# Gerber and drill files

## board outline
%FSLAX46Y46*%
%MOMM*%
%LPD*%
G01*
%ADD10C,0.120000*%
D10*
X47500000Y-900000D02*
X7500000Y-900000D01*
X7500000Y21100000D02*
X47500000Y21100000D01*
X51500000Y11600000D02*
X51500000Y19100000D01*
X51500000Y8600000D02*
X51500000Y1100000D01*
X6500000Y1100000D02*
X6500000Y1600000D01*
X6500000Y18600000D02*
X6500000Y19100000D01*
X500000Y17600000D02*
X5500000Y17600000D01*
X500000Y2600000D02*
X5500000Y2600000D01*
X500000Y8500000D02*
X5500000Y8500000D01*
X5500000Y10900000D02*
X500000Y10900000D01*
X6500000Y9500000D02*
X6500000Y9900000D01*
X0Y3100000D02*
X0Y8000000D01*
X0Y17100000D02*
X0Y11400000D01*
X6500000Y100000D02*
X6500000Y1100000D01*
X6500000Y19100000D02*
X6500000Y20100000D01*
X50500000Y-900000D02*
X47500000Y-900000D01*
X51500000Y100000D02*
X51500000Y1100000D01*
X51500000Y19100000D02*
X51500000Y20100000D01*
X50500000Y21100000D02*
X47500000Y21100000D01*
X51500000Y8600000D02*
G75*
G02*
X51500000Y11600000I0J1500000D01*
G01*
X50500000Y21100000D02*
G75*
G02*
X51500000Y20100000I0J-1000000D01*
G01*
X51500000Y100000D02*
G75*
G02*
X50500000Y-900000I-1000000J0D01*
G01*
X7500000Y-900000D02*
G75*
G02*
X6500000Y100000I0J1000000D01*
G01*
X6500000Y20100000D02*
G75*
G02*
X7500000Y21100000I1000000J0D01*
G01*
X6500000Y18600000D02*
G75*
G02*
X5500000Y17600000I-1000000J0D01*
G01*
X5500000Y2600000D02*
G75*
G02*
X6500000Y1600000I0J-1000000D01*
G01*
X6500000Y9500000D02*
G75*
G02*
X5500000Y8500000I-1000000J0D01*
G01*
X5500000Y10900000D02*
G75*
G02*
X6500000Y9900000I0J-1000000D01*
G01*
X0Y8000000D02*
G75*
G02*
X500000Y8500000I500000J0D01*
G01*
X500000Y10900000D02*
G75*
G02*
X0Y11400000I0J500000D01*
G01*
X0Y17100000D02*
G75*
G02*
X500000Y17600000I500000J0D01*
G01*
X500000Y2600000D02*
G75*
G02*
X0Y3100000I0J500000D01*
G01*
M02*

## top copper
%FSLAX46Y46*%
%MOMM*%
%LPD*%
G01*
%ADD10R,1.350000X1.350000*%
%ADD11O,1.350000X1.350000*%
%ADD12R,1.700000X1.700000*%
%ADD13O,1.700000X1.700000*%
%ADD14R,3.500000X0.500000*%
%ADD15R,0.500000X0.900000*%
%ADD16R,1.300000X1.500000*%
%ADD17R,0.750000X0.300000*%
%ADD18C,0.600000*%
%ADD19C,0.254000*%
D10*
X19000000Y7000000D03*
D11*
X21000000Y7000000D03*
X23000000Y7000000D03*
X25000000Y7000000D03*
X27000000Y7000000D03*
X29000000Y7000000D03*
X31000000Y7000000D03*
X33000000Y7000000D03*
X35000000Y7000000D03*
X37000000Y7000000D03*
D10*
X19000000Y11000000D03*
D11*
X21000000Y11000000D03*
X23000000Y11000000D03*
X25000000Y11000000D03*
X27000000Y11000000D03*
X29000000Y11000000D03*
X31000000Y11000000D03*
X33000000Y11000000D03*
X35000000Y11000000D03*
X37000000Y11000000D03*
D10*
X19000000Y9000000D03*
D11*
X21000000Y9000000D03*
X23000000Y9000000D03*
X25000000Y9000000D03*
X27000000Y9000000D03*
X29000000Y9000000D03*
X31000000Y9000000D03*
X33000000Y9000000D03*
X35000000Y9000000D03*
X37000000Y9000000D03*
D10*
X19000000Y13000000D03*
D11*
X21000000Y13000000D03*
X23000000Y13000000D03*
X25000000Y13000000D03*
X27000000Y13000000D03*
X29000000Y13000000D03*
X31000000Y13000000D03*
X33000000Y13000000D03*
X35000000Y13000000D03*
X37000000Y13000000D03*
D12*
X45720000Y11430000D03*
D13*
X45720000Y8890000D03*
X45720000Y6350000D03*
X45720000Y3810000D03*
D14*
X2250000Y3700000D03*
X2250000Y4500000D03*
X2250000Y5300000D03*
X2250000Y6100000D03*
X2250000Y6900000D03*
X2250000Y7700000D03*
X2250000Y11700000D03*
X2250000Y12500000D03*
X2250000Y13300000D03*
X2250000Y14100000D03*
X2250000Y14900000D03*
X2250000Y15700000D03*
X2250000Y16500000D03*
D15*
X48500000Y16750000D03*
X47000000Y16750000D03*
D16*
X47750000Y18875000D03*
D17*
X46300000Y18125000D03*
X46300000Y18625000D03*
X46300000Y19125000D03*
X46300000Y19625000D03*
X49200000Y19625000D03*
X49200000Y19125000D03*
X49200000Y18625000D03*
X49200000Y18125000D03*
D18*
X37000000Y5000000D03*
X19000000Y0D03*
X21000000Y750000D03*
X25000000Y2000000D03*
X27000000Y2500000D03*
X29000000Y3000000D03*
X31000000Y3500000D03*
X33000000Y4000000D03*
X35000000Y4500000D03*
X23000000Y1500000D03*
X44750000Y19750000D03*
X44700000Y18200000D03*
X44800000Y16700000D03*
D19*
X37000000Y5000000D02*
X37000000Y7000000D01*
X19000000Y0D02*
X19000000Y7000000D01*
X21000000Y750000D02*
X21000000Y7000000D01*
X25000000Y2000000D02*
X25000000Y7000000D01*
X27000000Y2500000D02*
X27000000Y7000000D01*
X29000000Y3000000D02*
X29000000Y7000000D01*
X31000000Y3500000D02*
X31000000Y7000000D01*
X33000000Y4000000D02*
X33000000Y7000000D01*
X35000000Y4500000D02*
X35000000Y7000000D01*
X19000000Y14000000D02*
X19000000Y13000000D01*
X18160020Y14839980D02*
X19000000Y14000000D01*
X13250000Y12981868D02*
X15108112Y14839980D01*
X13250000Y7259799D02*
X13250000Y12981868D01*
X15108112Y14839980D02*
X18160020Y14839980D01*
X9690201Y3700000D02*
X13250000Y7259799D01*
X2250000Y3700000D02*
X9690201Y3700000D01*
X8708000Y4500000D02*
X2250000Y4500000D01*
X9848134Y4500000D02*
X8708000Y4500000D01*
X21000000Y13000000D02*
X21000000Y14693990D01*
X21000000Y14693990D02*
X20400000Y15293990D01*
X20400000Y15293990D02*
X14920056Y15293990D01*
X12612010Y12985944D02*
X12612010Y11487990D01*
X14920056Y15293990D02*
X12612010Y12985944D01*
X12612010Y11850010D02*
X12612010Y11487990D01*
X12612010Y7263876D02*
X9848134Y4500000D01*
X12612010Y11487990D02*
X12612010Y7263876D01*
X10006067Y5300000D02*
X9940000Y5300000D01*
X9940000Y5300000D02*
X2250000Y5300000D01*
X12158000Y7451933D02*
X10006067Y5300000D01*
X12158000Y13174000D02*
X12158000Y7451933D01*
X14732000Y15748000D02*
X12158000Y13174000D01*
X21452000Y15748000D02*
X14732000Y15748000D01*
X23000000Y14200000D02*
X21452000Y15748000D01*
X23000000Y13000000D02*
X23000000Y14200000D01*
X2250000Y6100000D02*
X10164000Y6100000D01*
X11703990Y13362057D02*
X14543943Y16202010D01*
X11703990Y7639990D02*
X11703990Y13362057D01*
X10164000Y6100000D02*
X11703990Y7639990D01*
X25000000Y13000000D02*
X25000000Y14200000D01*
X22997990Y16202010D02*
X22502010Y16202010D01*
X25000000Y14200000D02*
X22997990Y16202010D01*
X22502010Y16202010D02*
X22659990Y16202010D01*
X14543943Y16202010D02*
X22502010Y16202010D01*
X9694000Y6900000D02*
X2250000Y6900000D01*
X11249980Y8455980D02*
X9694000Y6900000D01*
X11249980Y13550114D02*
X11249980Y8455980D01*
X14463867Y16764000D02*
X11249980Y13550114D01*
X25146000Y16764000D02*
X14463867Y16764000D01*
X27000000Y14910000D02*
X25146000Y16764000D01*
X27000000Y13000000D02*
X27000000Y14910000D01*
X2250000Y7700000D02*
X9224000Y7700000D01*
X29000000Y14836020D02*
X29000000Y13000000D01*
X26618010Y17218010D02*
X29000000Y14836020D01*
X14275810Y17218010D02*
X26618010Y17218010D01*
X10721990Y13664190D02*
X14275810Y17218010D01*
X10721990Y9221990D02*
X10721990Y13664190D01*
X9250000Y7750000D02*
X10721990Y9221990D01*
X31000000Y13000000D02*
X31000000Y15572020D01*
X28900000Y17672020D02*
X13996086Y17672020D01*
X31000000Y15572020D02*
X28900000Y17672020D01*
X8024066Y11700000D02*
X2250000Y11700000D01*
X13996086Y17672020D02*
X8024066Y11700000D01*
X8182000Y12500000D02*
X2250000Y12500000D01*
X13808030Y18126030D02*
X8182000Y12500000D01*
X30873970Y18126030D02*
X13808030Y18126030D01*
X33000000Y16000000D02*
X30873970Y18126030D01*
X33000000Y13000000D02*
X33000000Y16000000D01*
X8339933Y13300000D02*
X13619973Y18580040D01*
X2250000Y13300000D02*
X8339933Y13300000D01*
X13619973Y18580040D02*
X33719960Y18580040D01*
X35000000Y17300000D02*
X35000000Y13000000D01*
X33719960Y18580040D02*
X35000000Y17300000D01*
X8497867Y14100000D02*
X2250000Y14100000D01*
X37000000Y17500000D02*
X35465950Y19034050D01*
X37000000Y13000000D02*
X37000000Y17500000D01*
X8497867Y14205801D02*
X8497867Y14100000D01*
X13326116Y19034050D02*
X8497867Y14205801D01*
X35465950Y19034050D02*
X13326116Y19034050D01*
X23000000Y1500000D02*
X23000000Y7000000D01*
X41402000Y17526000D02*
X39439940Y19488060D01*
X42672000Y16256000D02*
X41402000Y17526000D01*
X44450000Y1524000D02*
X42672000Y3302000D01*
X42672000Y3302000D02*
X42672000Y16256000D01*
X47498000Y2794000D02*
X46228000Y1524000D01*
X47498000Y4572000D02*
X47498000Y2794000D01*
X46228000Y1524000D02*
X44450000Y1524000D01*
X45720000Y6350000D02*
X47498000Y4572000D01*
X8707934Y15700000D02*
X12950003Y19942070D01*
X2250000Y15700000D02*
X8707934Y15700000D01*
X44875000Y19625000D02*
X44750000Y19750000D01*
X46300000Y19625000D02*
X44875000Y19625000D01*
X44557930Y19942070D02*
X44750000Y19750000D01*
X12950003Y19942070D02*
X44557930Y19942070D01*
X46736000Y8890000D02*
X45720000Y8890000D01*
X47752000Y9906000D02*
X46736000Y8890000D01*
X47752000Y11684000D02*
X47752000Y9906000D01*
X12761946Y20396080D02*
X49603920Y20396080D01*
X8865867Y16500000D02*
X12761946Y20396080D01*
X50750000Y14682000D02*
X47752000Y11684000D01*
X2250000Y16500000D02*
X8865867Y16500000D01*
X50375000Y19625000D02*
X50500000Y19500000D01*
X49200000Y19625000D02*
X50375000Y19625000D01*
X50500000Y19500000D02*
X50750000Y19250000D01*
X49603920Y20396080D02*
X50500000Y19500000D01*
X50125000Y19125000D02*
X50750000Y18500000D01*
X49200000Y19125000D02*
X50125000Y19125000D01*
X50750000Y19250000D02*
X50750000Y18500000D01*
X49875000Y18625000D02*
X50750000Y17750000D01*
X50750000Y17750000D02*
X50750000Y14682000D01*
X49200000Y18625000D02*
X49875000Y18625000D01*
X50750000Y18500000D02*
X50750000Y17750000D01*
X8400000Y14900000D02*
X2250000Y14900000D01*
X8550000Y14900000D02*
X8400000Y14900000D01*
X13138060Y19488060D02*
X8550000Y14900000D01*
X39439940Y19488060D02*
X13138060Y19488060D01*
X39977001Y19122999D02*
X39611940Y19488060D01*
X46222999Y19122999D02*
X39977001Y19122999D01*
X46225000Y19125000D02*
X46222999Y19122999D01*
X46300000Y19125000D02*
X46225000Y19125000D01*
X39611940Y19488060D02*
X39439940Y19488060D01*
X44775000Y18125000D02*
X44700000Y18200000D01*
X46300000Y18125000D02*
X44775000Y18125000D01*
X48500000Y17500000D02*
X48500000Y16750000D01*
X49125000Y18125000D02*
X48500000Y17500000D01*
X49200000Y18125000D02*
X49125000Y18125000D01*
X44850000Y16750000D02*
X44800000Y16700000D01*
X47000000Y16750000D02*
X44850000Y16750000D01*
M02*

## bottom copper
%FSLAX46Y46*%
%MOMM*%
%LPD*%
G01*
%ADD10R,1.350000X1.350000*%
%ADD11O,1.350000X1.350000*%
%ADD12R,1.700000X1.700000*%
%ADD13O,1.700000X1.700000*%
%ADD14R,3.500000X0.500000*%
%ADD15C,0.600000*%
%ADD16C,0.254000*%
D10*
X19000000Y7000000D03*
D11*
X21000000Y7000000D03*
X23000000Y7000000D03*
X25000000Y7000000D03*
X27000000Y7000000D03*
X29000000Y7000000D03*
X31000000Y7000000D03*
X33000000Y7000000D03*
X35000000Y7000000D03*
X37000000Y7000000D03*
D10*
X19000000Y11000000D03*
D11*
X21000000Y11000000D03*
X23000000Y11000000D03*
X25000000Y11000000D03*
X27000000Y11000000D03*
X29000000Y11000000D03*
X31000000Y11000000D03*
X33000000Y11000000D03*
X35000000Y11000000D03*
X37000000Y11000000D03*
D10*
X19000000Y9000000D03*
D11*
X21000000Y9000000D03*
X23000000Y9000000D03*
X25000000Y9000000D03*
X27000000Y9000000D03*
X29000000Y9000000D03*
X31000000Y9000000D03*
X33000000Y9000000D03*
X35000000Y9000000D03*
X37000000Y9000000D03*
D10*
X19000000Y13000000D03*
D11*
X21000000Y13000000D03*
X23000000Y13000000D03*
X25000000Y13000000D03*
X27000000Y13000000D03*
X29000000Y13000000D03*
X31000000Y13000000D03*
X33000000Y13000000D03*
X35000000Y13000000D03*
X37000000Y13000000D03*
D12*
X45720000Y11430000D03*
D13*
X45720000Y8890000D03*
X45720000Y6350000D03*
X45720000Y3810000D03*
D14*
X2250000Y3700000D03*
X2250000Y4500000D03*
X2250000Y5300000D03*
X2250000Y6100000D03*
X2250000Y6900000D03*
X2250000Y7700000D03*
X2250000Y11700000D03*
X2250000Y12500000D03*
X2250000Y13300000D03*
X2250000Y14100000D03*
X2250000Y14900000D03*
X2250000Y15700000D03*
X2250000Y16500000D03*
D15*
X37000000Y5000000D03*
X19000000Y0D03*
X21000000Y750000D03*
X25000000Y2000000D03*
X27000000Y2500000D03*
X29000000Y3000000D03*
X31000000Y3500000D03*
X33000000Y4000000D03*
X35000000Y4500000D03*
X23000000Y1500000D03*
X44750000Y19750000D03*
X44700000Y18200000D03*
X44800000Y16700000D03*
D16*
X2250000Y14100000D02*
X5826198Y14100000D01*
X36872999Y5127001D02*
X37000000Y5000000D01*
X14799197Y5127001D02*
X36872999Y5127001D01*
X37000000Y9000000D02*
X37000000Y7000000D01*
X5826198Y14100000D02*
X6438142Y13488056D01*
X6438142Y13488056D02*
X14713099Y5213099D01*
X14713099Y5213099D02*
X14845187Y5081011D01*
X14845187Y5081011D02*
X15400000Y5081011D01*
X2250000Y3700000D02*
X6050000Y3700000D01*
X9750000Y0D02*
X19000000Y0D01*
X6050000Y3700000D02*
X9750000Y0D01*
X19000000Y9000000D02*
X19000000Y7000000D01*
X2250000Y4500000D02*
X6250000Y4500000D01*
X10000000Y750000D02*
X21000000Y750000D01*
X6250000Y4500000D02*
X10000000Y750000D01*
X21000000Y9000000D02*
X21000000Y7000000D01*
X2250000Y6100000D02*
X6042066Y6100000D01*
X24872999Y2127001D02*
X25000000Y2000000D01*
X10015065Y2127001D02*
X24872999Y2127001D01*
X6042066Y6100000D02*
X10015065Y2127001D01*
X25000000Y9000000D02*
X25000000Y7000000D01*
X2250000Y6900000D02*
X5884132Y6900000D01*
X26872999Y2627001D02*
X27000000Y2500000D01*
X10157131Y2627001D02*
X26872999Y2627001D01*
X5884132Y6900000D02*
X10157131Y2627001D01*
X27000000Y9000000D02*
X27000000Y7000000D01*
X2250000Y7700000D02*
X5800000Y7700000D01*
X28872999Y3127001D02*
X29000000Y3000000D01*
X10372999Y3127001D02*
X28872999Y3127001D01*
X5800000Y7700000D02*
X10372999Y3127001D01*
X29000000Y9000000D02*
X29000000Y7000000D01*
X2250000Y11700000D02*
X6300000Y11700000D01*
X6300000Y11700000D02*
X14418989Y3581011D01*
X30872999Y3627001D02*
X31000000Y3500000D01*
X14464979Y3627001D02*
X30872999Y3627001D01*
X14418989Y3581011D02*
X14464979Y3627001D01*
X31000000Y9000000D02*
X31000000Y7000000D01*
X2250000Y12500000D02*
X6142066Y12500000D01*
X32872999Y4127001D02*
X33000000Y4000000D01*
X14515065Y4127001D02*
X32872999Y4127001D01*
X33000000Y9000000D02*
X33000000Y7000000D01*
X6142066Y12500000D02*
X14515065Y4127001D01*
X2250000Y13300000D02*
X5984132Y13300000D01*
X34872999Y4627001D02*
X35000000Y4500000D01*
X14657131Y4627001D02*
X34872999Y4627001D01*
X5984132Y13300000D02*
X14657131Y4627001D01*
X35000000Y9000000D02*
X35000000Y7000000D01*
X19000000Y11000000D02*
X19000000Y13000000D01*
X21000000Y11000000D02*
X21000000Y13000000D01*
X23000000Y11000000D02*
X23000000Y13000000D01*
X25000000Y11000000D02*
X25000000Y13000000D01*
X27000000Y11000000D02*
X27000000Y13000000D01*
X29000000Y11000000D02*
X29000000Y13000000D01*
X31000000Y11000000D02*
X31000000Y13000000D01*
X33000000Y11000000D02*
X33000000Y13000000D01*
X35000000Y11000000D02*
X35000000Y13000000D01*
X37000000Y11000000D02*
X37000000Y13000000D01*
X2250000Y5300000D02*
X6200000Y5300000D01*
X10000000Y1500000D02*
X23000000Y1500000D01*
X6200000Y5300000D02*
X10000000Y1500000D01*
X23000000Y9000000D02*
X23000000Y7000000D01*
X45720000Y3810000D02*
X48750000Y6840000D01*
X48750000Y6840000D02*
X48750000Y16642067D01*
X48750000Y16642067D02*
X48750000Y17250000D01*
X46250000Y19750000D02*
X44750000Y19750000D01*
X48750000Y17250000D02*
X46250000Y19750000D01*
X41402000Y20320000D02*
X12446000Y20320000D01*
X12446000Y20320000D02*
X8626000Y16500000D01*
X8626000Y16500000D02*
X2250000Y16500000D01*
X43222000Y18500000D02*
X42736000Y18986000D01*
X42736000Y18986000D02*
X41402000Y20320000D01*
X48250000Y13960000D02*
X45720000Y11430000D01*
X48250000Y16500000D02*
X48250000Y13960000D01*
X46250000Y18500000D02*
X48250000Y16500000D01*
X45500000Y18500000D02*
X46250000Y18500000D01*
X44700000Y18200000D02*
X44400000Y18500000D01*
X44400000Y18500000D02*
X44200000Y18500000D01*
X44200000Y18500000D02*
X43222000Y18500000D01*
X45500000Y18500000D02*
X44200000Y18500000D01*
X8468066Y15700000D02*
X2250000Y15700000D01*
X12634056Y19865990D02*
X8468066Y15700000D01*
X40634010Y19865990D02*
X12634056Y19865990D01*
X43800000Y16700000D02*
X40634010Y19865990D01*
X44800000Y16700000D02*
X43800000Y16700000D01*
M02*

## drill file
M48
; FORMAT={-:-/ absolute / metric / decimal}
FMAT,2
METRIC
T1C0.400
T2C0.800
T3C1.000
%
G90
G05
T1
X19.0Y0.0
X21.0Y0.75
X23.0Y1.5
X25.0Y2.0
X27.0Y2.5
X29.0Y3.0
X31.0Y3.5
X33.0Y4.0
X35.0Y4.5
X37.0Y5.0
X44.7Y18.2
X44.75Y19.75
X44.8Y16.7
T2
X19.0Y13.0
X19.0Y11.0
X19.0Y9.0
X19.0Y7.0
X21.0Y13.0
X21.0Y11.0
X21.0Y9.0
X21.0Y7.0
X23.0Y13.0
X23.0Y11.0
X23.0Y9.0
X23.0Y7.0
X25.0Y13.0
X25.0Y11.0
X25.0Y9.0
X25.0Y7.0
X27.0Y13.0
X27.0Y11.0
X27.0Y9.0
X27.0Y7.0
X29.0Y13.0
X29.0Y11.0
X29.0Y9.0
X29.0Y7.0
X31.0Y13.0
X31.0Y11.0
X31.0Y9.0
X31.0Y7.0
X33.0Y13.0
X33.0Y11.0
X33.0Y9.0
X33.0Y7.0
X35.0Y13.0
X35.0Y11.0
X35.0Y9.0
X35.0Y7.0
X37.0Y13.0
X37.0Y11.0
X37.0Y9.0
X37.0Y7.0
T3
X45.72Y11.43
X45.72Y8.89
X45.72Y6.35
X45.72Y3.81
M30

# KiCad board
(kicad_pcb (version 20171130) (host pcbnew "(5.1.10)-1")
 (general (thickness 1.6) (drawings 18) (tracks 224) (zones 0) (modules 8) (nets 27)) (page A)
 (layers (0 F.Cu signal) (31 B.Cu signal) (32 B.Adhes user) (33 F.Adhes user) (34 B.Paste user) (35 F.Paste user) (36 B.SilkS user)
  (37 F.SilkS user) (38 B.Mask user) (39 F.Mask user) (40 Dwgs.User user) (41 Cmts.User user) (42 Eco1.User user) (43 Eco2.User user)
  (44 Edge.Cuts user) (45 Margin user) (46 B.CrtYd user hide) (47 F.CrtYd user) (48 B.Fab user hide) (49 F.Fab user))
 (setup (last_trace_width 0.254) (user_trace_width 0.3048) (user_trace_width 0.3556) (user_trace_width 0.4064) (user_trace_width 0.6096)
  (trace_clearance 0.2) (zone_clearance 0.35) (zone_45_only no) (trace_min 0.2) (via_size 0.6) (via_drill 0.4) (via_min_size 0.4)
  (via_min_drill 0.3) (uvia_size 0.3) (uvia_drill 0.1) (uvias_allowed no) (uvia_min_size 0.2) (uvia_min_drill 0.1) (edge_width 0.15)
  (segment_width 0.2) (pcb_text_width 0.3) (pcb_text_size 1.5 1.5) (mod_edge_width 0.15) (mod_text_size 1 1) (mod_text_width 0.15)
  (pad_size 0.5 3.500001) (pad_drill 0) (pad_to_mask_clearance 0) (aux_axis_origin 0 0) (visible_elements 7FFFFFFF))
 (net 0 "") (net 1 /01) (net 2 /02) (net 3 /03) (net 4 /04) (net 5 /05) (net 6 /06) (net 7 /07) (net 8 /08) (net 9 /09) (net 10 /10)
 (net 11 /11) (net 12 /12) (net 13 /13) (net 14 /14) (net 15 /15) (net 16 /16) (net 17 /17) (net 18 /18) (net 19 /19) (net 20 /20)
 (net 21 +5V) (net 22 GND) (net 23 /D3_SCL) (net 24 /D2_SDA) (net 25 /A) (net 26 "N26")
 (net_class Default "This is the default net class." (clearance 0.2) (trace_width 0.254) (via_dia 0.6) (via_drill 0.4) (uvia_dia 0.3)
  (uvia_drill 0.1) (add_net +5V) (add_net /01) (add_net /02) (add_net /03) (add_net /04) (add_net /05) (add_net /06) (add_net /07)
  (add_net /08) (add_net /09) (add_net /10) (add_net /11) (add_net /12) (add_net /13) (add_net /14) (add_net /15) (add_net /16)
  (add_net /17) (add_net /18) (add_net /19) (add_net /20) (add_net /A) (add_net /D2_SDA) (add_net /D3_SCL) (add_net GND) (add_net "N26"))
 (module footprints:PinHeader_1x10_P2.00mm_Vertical (layer F.Cu) (at 19 -7 90)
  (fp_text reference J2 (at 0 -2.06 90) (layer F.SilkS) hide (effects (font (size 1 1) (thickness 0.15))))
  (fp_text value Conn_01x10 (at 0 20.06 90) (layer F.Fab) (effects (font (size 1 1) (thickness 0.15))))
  (pad 1 thru_hole rect (at 0 0 90) (size 1.35 1.35) (drill 0.8) (layers *.Cu *.Mask) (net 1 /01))
  (pad 2 thru_hole oval (at 0 2 90) (size 1.35 1.35) (drill 0.8) (layers *.Cu *.Mask) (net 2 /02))
  (pad 3 thru_hole oval (at 0 4 90) (size 1.35 1.35) (drill 0.8) (layers *.Cu *.Mask) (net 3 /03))
  (pad 4 thru_hole oval (at 0 6 90) (size 1.35 1.35) (drill 0.8) (layers *.Cu *.Mask) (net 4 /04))
  (pad 5 thru_hole oval (at 0 8 90) (size 1.35 1.35) (drill 0.8) (layers *.Cu *.Mask) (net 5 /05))
  (pad 6 thru_hole oval (at 0 10 90) (size 1.35 1.35) (drill 0.8) (layers *.Cu *.Mask) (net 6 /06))
  (pad 7 thru_hole oval (at 0 12 90) (size 1.35 1.35) (drill 0.8) (layers *.Cu *.Mask) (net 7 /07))
  (pad 8 thru_hole oval (at 0 14 90) (size 1.35 1.35) (drill 0.8) (layers *.Cu *.Mask) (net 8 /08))
  (pad 9 thru_hole oval (at 0 16 90) (size 1.35 1.35) (drill 0.8) (layers *.Cu *.Mask) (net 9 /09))
  (pad 10 thru_hole oval (at 0 18 90) (size 1.35 1.35) (drill 0.8) (layers *.Cu *.Mask) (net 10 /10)))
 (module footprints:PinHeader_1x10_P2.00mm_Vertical (layer F.Cu) (at 19 -11 90)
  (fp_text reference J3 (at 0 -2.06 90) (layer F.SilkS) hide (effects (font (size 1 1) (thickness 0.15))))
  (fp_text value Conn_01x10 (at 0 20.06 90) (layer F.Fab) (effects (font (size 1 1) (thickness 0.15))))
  (pad 1 thru_hole rect (at 0 0 90) (size 1.35 1.35) (drill 0.8) (layers *.Cu *.Mask) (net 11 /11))
  (pad 2 thru_hole oval (at 0 2 90) (size 1.35 1.35) (drill 0.8) (layers *.Cu *.Mask) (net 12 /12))
  (pad 3 thru_hole oval (at 0 4 90) (size 1.35 1.35) (drill 0.8) (layers *.Cu *.Mask) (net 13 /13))
  (pad 4 thru_hole oval (at 0 6 90) (size 1.35 1.35) (drill 0.8) (layers *.Cu *.Mask) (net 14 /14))
  (pad 5 thru_hole oval (at 0 8 90) (size 1.35 1.35) (drill 0.8) (layers *.Cu *.Mask) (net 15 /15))
  (pad 6 thru_hole oval (at 0 10 90) (size 1.35 1.35) (drill 0.8) (layers *.Cu *.Mask) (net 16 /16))
  (pad 7 thru_hole oval (at 0 12 90) (size 1.35 1.35) (drill 0.8) (layers *.Cu *.Mask) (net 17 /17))
  (pad 8 thru_hole oval (at 0 14 90) (size 1.35 1.35) (drill 0.8) (layers *.Cu *.Mask) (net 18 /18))
  (pad 9 thru_hole oval (at 0 16 90) (size 1.35 1.35) (drill 0.8) (layers *.Cu *.Mask) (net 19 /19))
  (pad 10 thru_hole oval (at 0 18 90) (size 1.35 1.35) (drill 0.8) (layers *.Cu *.Mask) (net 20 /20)))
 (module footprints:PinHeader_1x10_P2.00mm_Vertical (layer F.Cu) (at 19 -9 90)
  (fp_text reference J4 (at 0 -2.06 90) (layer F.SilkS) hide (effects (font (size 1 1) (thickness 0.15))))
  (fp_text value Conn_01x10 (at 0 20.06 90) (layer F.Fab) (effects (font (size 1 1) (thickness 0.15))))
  (pad 1 thru_hole rect (at 0 0 90) (size 1.35 1.35) (drill 0.8) (layers *.Cu *.Mask) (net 1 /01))
  (pad 2 thru_hole oval (at 0 2 90) (size 1.35 1.35) (drill 0.8) (layers *.Cu *.Mask) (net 2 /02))
  (pad 3 thru_hole oval (at 0 4 90) (size 1.35 1.35) (drill 0.8) (layers *.Cu *.Mask) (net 3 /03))
  (pad 4 thru_hole oval (at 0 6 90) (size 1.35 1.35) (drill 0.8) (layers *.Cu *.Mask) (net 4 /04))
  (pad 5 thru_hole oval (at 0 8 90) (size 1.35 1.35) (drill 0.8) (layers *.Cu *.Mask) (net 5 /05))
  (pad 6 thru_hole oval (at 0 10 90) (size 1.35 1.35) (drill 0.8) (layers *.Cu *.Mask) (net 6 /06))
  (pad 7 thru_hole oval (at 0 12 90) (size 1.35 1.35) (drill 0.8) (layers *.Cu *.Mask) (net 7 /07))
  (pad 8 thru_hole oval (at 0 14 90) (size 1.35 1.35) (drill 0.8) (layers *.Cu *.Mask) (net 8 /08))
  (pad 9 thru_hole oval (at 0 16 90) (size 1.35 1.35) (drill 0.8) (layers *.Cu *.Mask) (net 9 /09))
  (pad 10 thru_hole oval (at 0 18 90) (size 1.35 1.35) (drill 0.8) (layers *.Cu *.Mask) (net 10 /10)))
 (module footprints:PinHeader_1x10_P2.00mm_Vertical (layer F.Cu) (at 19 -13 90)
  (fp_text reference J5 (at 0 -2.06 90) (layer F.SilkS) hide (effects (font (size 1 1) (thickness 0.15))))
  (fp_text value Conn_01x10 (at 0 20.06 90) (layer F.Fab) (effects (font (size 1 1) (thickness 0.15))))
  (pad 1 thru_hole rect (at 0 0 90) (size 1.35 1.35) (drill 0.8) (layers *.Cu *.Mask) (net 11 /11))
  (pad 2 thru_hole oval (at 0 2 90) (size 1.35 1.35) (drill 0.8) (layers *.Cu *.Mask) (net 12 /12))
  (pad 3 thru_hole oval (at 0 4 90) (size 1.35 1.35) (drill 0.8) (layers *.Cu *.Mask) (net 13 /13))
  (pad 4 thru_hole oval (at 0 6 90) (size 1.35 1.35) (drill 0.8) (layers *.Cu *.Mask) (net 14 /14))
  (pad 5 thru_hole oval (at 0 8 90) (size 1.35 1.35) (drill 0.8) (layers *.Cu *.Mask) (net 15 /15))
  (pad 6 thru_hole oval (at 0 10 90) (size 1.35 1.35) (drill 0.8) (layers *.Cu *.Mask) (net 16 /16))
  (pad 7 thru_hole oval (at 0 12 90) (size 1.35 1.35) (drill 0.8) (layers *.Cu *.Mask) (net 17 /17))
  (pad 8 thru_hole oval (at 0 14 90) (size 1.35 1.35) (drill 0.8) (layers *.Cu *.Mask) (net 18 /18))
  (pad 9 thru_hole oval (at 0 16 90) (size 1.35 1.35) (drill 0.8) (layers *.Cu *.Mask) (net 19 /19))
  (pad 10 thru_hole oval (at 0 18 90) (size 1.35 1.35) (drill 0.8) (layers *.Cu *.Mask) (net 20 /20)))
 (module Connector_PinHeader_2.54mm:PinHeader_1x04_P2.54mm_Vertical (layer F.Cu) (at 45.72 -11.43)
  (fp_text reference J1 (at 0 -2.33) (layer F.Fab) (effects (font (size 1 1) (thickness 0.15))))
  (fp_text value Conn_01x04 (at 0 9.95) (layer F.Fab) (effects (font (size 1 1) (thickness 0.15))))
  (pad 1 thru_hole rect (at 0 0) (size 1.7 1.7) (drill 1) (layers *.Cu *.Mask) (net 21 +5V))
  (pad 2 thru_hole oval (at 0 2.54) (size 1.7 1.7) (drill 1) (layers *.Cu *.Mask) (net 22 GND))
  (pad 3 thru_hole oval (at 0 5.08) (size 1.7 1.7) (drill 1) (layers *.Cu *.Mask) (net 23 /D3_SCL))
  (pad 4 thru_hole oval (at 0 7.62) (size 1.7 1.7) (drill 1) (layers *.Cu *.Mask) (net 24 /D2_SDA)))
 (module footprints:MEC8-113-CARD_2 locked (layer F.Cu) (at 0 -0.1 90)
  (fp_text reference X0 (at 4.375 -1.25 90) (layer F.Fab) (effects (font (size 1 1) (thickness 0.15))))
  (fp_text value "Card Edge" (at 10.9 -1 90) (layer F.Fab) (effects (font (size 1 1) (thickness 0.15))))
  (fp_line (start -1 47.5) (end -1 7.5) (layer Edge.Cuts) (width 0.12))
  (fp_line (start 21 7.5) (end 21 47.5) (layer Edge.Cuts) (width 0.12))
  (fp_line (start 11.5 51.5) (end 19 51.5) (layer Edge.Cuts) (width 0.12))
  (fp_line (start 8.5 51.5) (end 1 51.5) (layer Edge.Cuts) (width 0.12))
  (fp_line (start 1 6.5) (end 1.5 6.5) (layer Edge.Cuts) (width 0.12))
  (fp_line (start 18.5 6.5) (end 19 6.5) (layer Edge.Cuts) (width 0.12))
  (fp_line (start 17.5 0.5) (end 17.5 5.5) (layer Edge.Cuts) (width 0.12))
  (fp_line (start 2.5 0.5) (end 2.5 5.5) (layer Edge.Cuts) (width 0.12))
  (fp_line (start 8.4 0.5) (end 8.4 5.5) (layer Edge.Cuts) (width 0.12))
  (fp_line (start 10.8 5.5) (end 10.8 0.5) (layer Edge.Cuts) (width 0.12))
  (fp_line (start 9.4 6.5) (end 9.8 6.5) (layer Edge.Cuts) (width 0.12))
  (fp_line (start 3 0) (end 7.9 0) (layer Edge.Cuts) (width 0.12))
  (fp_line (start 17 0) (end 11.3 0) (layer Edge.Cuts) (width 0.12))
  (fp_line (start 0 6.5) (end 1 6.5) (layer Edge.Cuts) (width 0.12))
  (fp_line (start 19 6.5) (end 20 6.5) (layer Edge.Cuts) (width 0.12))
  (fp_line (start -1 50.5) (end -1 47.5) (layer Edge.Cuts) (width 0.12))
  (fp_line (start 0 51.5) (end 1 51.5) (layer Edge.Cuts) (width 0.12))
  (fp_line (start 19 51.5) (end 20 51.5) (layer Edge.Cuts) (width 0.12))
  (fp_line (start 21 50.5) (end 21 47.5) (layer Edge.Cuts) (width 0.12))
  (fp_arc (start 10 51.5) (end 11.5 51.5) (angle -180) (layer Edge.Cuts) (width 0.12))
  (fp_arc (start 20 50.5) (end 20 51.5) (angle -90) (layer Edge.Cuts) (width 0.12))
  (fp_arc (start 0 50.5) (end -1 50.5) (angle -90) (layer Edge.Cuts) (width 0.12))
  (fp_arc (start 0 7.5) (end 0 6.5) (angle -90) (layer Edge.Cuts) (width 0.12))
  (fp_arc (start 20 7.5) (end 21 7.5) (angle -90) (layer Edge.Cuts) (width 0.12))
  (fp_arc (start 18.5 5.5) (end 17.5 5.5) (angle -90) (layer Edge.Cuts) (width 0.12))
  (fp_arc (start 1.5 5.5) (end 1.5 6.5) (angle -90) (layer Edge.Cuts) (width 0.12))
  (fp_arc (start 9.4 5.5) (end 8.4 5.5) (angle -90) (layer Edge.Cuts) (width 0.12))
  (fp_arc (start 9.8 5.5) (end 9.8 6.5) (angle -90) (layer Edge.Cuts) (width 0.12))
  (fp_arc (start 7.9 0.5) (end 8.4 0.5) (angle -90) (layer Edge.Cuts) (width 0.12))
  (fp_arc (start 11.3 0.5) (end 11.3 0) (angle -90) (layer Edge.Cuts) (width 0.12))
  (fp_arc (start 17 0.5) (end 17.5 0.5) (angle -90) (layer Edge.Cuts) (width 0.12))
  (fp_arc (start 3 0.5) (end 3 0) (angle -90) (layer Edge.Cuts) (width 0.12))
  (pad 14 smd rect (at 3.6 2.25 90) (size 0.5 3.5) (layers F.Cu F.Paste F.Mask) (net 11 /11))
  (pad 1 smd rect (at 3.6 2.25 90) (size 0.5 3.5) (layers B.Cu B.Paste B.Mask) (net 1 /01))
  (pad 15 smd rect (at 4.4 2.25 90) (size 0.5 3.5) (layers F.Cu F.Paste F.Mask) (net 12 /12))
  (pad 2 smd rect (at 4.4 2.25 90) (size 0.5 3.5) (layers B.Cu B.Paste B.Mask) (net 2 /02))
  (pad 16 smd rect (at 5.2 2.25 90) (size 0.5 3.5) (layers F.Cu F.Paste F.Mask) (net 13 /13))
  (pad 3 smd rect (at 5.2 2.25 90) (size 0.5 3.5) (layers B.Cu B.Paste B.Mask) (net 3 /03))
  (pad 17 smd rect (at 6 2.25 90) (size 0.5 3.5) (layers F.Cu F.Paste F.Mask) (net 14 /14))
  (pad 4 smd rect (at 6 2.25 90) (size 0.5 3.5) (layers B.Cu B.Paste B.Mask) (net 4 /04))
  (pad 18 smd rect (at 6.8 2.25 90) (size 0.5 3.5) (layers F.Cu F.Paste F.Mask) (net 15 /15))
  (pad 5 smd rect (at 6.8 2.25 90) (size 0.5 3.5) (layers B.Cu B.Paste B.Mask) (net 5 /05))
  (pad 19 smd rect (at 7.6 2.25 90) (size 0.5 3.5) (layers F.Cu F.Paste F.Mask) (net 16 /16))
  (pad 6 smd rect (at 7.6 2.25 90) (size 0.5 3.5) (layers B.Cu B.Paste B.Mask) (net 6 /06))
  (pad 20 smd rect (at 11.6 2.25 90) (size 0.5 3.5) (layers F.Cu F.Paste F.Mask) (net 17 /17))
  (pad 7 smd rect (at 11.6 2.25 90) (size 0.5 3.5) (layers B.Cu B.Paste B.Mask) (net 7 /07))
  (pad 21 smd rect (at 12.4 2.25 90) (size 0.5 3.5) (layers F.Cu F.Paste F.Mask) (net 18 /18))
  (pad 8 smd rect (at 12.4 2.25 90) (size 0.5 3.5) (layers B.Cu B.Paste B.Mask) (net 8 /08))
  (pad 22 smd rect (at 13.2 2.25 90) (size 0.5 3.5) (layers F.Cu F.Paste F.Mask) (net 19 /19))
  (pad 9 smd rect (at 13.2 2.25 90) (size 0.5 3.5) (layers B.Cu B.Paste B.Mask) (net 9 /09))
  (pad 23 smd rect (at 14 2.25 90) (size 0.5 3.5) (layers F.Cu F.Paste F.Mask) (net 20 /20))
  (pad 10 smd rect (at 14 2.25 90) (size 0.5 3.5) (layers B.Cu B.Paste B.Mask) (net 10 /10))
  (pad 24 smd rect (at 14.8 2.25 90) (size 0.5 3.5) (layers F.Cu F.Paste F.Mask) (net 23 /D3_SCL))
  (pad 11 smd rect (at 14.8 2.25 90) (size 0.5 3.5) (layers B.Cu B.Paste B.Mask))
  (pad 25 smd rect (at 15.6 2.25 90) (size 0.5 3.5) (layers F.Cu F.Paste F.Mask) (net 24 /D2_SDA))
  (pad 12 smd rect (at 15.6 2.25 90) (size 0.5 3.5) (layers B.Cu B.Paste B.Mask) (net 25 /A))
  (pad 26 smd rect (at 16.4 2.25 90) (size 0.5 3.5) (layers F.Cu F.Paste F.Mask) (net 22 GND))
  (pad 13 smd rect (at 16.4 2.25 90) (size 0.5 3.5) (layers B.Cu B.Paste B.Mask) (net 21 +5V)))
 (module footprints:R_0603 (layer F.Cu) (at 47.75 -16.75 180)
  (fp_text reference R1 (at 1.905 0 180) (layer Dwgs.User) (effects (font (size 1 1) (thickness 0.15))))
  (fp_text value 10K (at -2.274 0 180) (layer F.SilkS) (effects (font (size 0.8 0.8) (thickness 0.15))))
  (pad 1 smd rect (at -0.75 0 180) (size 0.5 0.9) (layers F.Cu F.Paste F.Mask) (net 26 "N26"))
  (pad 2 smd rect (at 0.75 0 180) (size 0.5 0.9) (layers F.Cu F.Paste F.Mask) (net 25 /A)))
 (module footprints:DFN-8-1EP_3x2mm (layer F.Cu) (at 47.75 -18.875 180)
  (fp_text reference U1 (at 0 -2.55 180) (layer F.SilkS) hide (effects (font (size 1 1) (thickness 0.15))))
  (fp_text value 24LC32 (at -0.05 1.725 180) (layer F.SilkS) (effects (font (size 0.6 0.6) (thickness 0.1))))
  (pad "" smd rect (at 0.325 0.375 180) (size 0.5 0.6) (layers F.Paste))
  (pad "" smd rect (at 0.325 -0.375 180) (size 0.5 0.6) (layers F.Paste))
  (pad "" smd rect (at -0.325 0.375 180) (size 0.5 0.6) (layers F.Paste))
  (pad "" smd rect (at -0.325 -0.375 180) (size 0.5 0.6) (layers F.Paste))
  (pad 9 smd rect (at 0 0 180) (size 1.3 1.5) (layers F.Cu F.Mask))
  (pad 8 smd rect (at 1.45 -0.75 180) (size 0.75 0.3) (layers F.Cu F.Paste F.Mask) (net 21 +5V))
  (pad 7 smd rect (at 1.45 -0.25 180) (size 0.75 0.3) (layers F.Cu F.Paste F.Mask))
  (pad 6 smd rect (at 1.45 0.25 180) (size 0.75 0.3) (layers F.Cu F.Paste F.Mask) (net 23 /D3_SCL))
  (pad 5 smd rect (at 1.45 0.75 180) (size 0.75 0.3) (layers F.Cu F.Paste F.Mask) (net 24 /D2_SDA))
  (pad 4 smd rect (at -1.45 0.75 180) (size 0.75 0.3) (layers F.Cu F.Paste F.Mask) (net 22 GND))
  (pad 3 smd rect (at -1.45 0.25 180) (size 0.75 0.3) (layers F.Cu F.Paste F.Mask) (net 22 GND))
  (pad 2 smd rect (at -1.45 -0.25 180) (size 0.75 0.3) (layers F.Cu F.Paste F.Mask) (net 22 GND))
  (pad 1 smd rect (at -1.45 -0.75 180) (size 0.75 0.3) (layers F.Cu F.Paste F.Mask) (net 26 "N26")))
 (segment (start 2.25 -14.1) (end 5.826198 -14.1) (width 0.254) (layer B.Cu) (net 10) (status 10))
 (via (at 37 -5) (size 0.6) (drill 0.4) (layers F.Cu B.Cu) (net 10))
 (segment (start 36.872999 -5.127001) (end 37 -5) (width 0.254) (layer B.Cu) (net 10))
 (segment (start 14.799197 -5.127001) (end 36.872999 -5.127001) (width 0.254) (layer B.Cu) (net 10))
 (segment (start 37 -5) (end 37 -7) (width 0.254) (layer F.Cu) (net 10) (status 20))
 (segment (start 37 -9) (end 37 -7) (width 0.254) (layer B.Cu) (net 10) (status 30))
 (segment (start 5.826198 -14.1) (end 6.438142 -13.488056) (width 0.254) (layer B.Cu) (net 10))
 (segment (start 6.438142 -13.488056) (end 14.713099 -5.213099) (width 0.254) (layer B.Cu) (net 10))
 (segment (start 14.713099 -5.213099) (end 14.845187 -5.081011) (width 0.254) (layer B.Cu) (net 10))
 (segment (start 14.845187 -5.081011) (end 15.4 -5.081011) (width 0.254) (layer B.Cu) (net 10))
 (segment (start 2.25 -3.7) (end 6.05 -3.7) (width 0.254) (layer B.Cu) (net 1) (status 10))
 (via (at 19 0) (size 0.6) (drill 0.4) (layers F.Cu B.Cu) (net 1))
 (segment (start 9.75 0) (end 19 0) (width 0.254) (layer B.Cu) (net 1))
 (segment (start 6.05 -3.7) (end 9.75 0) (width 0.254) (layer B.Cu) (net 1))
 (segment (start 19 0) (end 19 -7) (width 0.254) (layer F.Cu) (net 1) (status 20))
 (segment (start 19 -9) (end 19 -7) (width 0.254) (layer B.Cu) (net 1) (status 30))
 (segment (start 2.25 -4.5) (end 6.25 -4.5) (width 0.254) (layer B.Cu) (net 2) (status 10))
 (via (at 21 -0.75) (size 0.6) (drill 0.4) (layers F.Cu B.Cu) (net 2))
 (segment (start 10 -0.75) (end 21 -0.75) (width 0.254) (layer B.Cu) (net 2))
 (segment (start 6.25 -4.5) (end 10 -0.75) (width 0.254) (layer B.Cu) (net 2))
 (segment (start 21 -0.75) (end 21 -7) (width 0.254) (layer F.Cu) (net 2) (status 20))
 (segment (start 21 -9) (end 21 -7) (width 0.254) (layer B.Cu) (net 2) (status 30))
 (segment (start 2.25 -6.1) (end 6.042066 -6.1) (width 0.254) (layer B.Cu) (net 4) (status 10))
 (via (at 25 -2) (size 0.6) (drill 0.4) (layers F.Cu B.Cu) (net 4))
 (segment (start 24.872999 -2.127001) (end 25 -2) (width 0.254) (layer B.Cu) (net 4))
 (segment (start 10.015065 -2.127001) (end 24.872999 -2.127001) (width 0.254) (layer B.Cu) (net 4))
 (segment (start 6.042066 -6.1) (end 10.015065 -2.127001) (width 0.254) (layer B.Cu) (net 4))
 (segment (start 25 -2) (end 25 -7) (width 0.254) (layer F.Cu) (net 4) (status 20))
 (segment (start 25 -9) (end 25 -7) (width 0.254) (layer B.Cu) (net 4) (status 30))
 (segment (start 2.25 -6.9) (end 5.884132 -6.9) (width 0.254) (layer B.Cu) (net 5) (status 10))
 (via (at 27 -2.5) (size 0.6) (drill 0.4) (layers F.Cu B.Cu) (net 5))
 (segment (start 26.872999 -2.627001) (end 27 -2.5) (width 0.254) (layer B.Cu) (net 5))
 (segment (start 10.157131 -2.627001) (end 26.872999 -2.627001) (width 0.254) (layer B.Cu) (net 5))
 (segment (start 5.884132 -6.9) (end 10.157131 -2.627001) (width 0.254) (layer B.Cu) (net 5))
 (segment (start 27 -2.5) (end 27 -7) (width 0.254) (layer F.Cu) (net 5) (status 20))
 (segment (start 27 -9) (end 27 -7) (width 0.254) (layer B.Cu) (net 5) (status 30))
 (segment (start 2.25 -7.7) (end 5.8 -7.7) (width 0.254) (layer B.Cu) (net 6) (status 10))
 (via (at 29 -3) (size 0.6) (drill 0.4) (layers F.Cu B.Cu) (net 6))
 (segment (start 28.872999 -3.127001) (end 29 -3) (width 0.254) (layer B.Cu) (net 6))
 (segment (start 10.372999 -3.127001) (end 28.872999 -3.127001) (width 0.254) (layer B.Cu) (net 6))
 (segment (start 5.8 -7.7) (end 10.372999 -3.127001) (width 0.254) (layer B.Cu) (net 6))
 (segment (start 29 -3) (end 29 -7) (width 0.254) (layer F.Cu) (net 6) (status 20))
 (segment (start 29 -9) (end 29 -7) (width 0.254) (layer B.Cu) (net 6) (status 30))
 (segment (start 2.25 -11.7) (end 6.3 -11.7) (width 0.254) (layer B.Cu) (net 7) (status 10))
 (segment (start 6.3 -11.7) (end 14.418989 -3.581011) (width 0.254) (layer B.Cu) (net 7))
 (via (at 31 -3.5) (size 0.6) (drill 0.4) (layers F.Cu B.Cu) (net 7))
 (segment (start 30.872999 -3.627001) (end 31 -3.5) (width 0.254) (layer B.Cu) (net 7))
 (segment (start 14.464979 -3.627001) (end 30.872999 -3.627001) (width 0.254) (layer B.Cu) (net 7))
 (segment (start 14.418989 -3.581011) (end 14.464979 -3.627001) (width 0.254) (layer B.Cu) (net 7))
 (segment (start 31 -3.5) (end 31 -7) (width 0.254) (layer F.Cu) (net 7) (status 20))
 (segment (start 31 -9) (end 31 -7) (width 0.254) (layer B.Cu) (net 7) (status 30))
 (segment (start 2.25 -12.5) (end 6.142066 -12.5) (width 0.254) (layer B.Cu) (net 8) (status 10))
 (via (at 33 -4) (size 0.6) (drill 0.4) (layers F.Cu B.Cu) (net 8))
 (segment (start 32.872999 -4.127001) (end 33 -4) (width 0.254) (layer B.Cu) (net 8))
 (segment (start 14.515065 -4.127001) (end 32.872999 -4.127001) (width 0.254) (layer B.Cu) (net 8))
 (segment (start 33 -4) (end 33 -7) (width 0.254) (layer F.Cu) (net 8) (status 20))
 (segment (start 33 -9) (end 33 -7) (width 0.254) (layer B.Cu) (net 8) (status 30))
 (segment (start 6.142066 -12.5) (end 14.515065 -4.127001) (width 0.254) (layer B.Cu) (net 8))
 (segment (start 2.25 -13.3) (end 5.984132 -13.3) (width 0.254) (layer B.Cu) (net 9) (status 10))
 (via (at 35 -4.5) (size 0.6) (drill 0.4) (layers F.Cu B.Cu) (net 9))
 (segment (start 34.872999 -4.627001) (end 35 -4.5) (width 0.254) (layer B.Cu) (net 9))
 (segment (start 14.657131 -4.627001) (end 34.872999 -4.627001) (width 0.254) (layer B.Cu) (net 9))
 (segment (start 5.984132 -13.3) (end 14.657131 -4.627001) (width 0.254) (layer B.Cu) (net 9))
 (segment (start 35 -4.5) (end 35 -7) (width 0.254) (layer F.Cu) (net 9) (status 20))
 (segment (start 35 -9) (end 35 -7) (width 0.254) (layer B.Cu) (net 9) (status 30))
 (segment (start 19 -11) (end 19 -13) (width 0.254) (layer B.Cu) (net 11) (status 30))
 (segment (start 19 -14) (end 19 -13) (width 0.254) (layer F.Cu) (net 11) (status 20))
 (segment (start 18.16002 -14.83998) (end 19 -14) (width 0.254) (layer F.Cu) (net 11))
 (segment (start 13.25 -12.981868) (end 15.108112 -14.83998) (width 0.254) (layer F.Cu) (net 11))
 (segment (start 13.25 -7.259799) (end 13.25 -12.981868) (width 0.254) (layer F.Cu) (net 11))
 (segment (start 15.108112 -14.83998) (end 18.16002 -14.83998) (width 0.254) (layer F.Cu) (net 11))
 (segment (start 9.690201 -3.7) (end 13.25 -7.259799) (width 0.254) (layer F.Cu) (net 11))
 (segment (start 2.25 -3.7) (end 9.690201 -3.7) (width 0.254) (layer F.Cu) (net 11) (status 10))
 (segment (start 8.708 -4.5) (end 2.25 -4.5) (width 0.254) (layer F.Cu) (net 12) (status 20))
 (segment (start 9.848134 -4.5) (end 8.708 -4.5) (width 0.254) (layer F.Cu) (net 12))
 (segment (start 21 -13) (end 21 -14.69399) (width 0.254) (layer F.Cu) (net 12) (status 10))
 (segment (start 21 -14.69399) (end 20.4 -15.29399) (width 0.254) (layer F.Cu) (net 12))
 (segment (start 20.4 -15.29399) (end 14.920056 -15.29399) (width 0.254) (layer F.Cu) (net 12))
 (segment (start 12.61201 -12.985944) (end 12.61201 -11.48799) (width 0.254) (layer F.Cu) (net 12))
 (segment (start 14.920056 -15.29399) (end 12.61201 -12.985944) (width 0.254) (layer F.Cu) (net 12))
 (segment (start 12.61201 -11.85001) (end 12.61201 -11.48799) (width 0.254) (layer F.Cu) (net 12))
 (segment (start 21 -11) (end 21 -13) (width 0.254) (layer B.Cu) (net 12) (status 30))
 (segment (start 12.61201 -7.263876) (end 9.848134 -4.5) (width 0.254) (layer F.Cu) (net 12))
 (segment (start 12.61201 -11.48799) (end 12.61201 -7.263876) (width 0.254) (layer F.Cu) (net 12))
 (segment (start 10.006067 -5.3) (end 9.94 -5.3) (width 0.254) (layer F.Cu) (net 13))
 (segment (start 9.94 -5.3) (end 2.25 -5.3) (width 0.254) (layer F.Cu) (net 13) (status 20))
 (segment (start 12.158 -7.451933) (end 10.006067 -5.3) (width 0.254) (layer F.Cu) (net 13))
 (segment (start 12.158 -13.174) (end 12.158 -7.451933) (width 0.254) (layer F.Cu) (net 13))
 (segment (start 14.732 -15.748) (end 12.158 -13.174) (width 0.254) (layer F.Cu) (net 13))
 (segment (start 21.452 -15.748) (end 14.732 -15.748) (width 0.254) (layer F.Cu) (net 13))
 (segment (start 23 -14.2) (end 21.452 -15.748) (width 0.254) (layer F.Cu) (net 13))
 (segment (start 23 -13) (end 23 -14.2) (width 0.254) (layer F.Cu) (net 13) (status 10))
 (segment (start 23 -11) (end 23 -13) (width 0.254) (layer B.Cu) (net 13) (status 30))
 (segment (start 2.25 -6.1) (end 10.164 -6.1) (width 0.254) (layer F.Cu) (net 14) (status 10))
 (segment (start 11.70399 -13.362057) (end 14.543943 -16.20201) (width 0.254) (layer F.Cu) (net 14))
 (segment (start 11.70399 -7.63999) (end 11.70399 -13.362057) (width 0.254) (layer F.Cu) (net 14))
 (segment (start 10.164 -6.1) (end 11.70399 -7.63999) (width 0.254) (layer F.Cu) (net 14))
 (segment (start 25 -13) (end 25 -14.2) (width 0.254) (layer F.Cu) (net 14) (status 10))
 (segment (start 22.99799 -16.20201) (end 22.50201 -16.20201) (width 0.254) (layer F.Cu) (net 14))
 (segment (start 25 -14.2) (end 22.99799 -16.20201) (width 0.254) (layer F.Cu) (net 14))
 (segment (start 22.50201 -16.20201) (end 22.65999 -16.20201) (width 0.254) (layer F.Cu) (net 14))
 (segment (start 14.543943 -16.20201) (end 22.50201 -16.20201) (width 0.254) (layer F.Cu) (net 14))
 (segment (start 25 -11) (end 25 -13) (width 0.254) (layer B.Cu) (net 14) (status 30))
 (segment (start 27 -11) (end 27 -13) (width 0.254) (layer B.Cu) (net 15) (status 30))
 (segment (start 9.694 -6.9) (end 2.25 -6.9) (width 0.254) (layer F.Cu) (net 15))
 (segment (start 11.24998 -8.45598) (end 9.694 -6.9) (width 0.254) (layer F.Cu) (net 15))
 (segment (start 11.24998 -13.550114) (end 11.24998 -8.45598) (width 0.254) (layer F.Cu) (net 15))
 (segment (start 14.463867 -16.764) (end 11.24998 -13.550114) (width 0.254) (layer F.Cu) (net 15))
 (segment (start 25.146 -16.764) (end 14.463867 -16.764) (width 0.254) (layer F.Cu) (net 15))
 (segment (start 27 -14.91) (end 25.146 -16.764) (width 0.254) (layer F.Cu) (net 15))
 (segment (start 27 -13) (end 27 -14.91) (width 0.254) (layer F.Cu) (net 15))
 (segment (start 2.25 -7.7) (end 9.224 -7.7) (width 0.254) (layer F.Cu) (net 16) (status 10))
 (segment (start 29 -11) (end 29 -13) (width 0.254) (layer B.Cu) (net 16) (status 30))
 (segment (start 29 -14.83602) (end 29 -13) (width 0.254) (layer F.Cu) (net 16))
 (segment (start 26.61801 -17.21801) (end 29 -14.83602) (width 0.254) (layer F.Cu) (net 16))
 (segment (start 14.27581 -17.21801) (end 26.61801 -17.21801) (width 0.254) (layer F.Cu) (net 16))
 (segment (start 10.72199 -13.66419) (end 14.27581 -17.21801) (width 0.254) (layer F.Cu) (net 16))
 (segment (start 10.72199 -9.22199) (end 10.72199 -13.66419) (width 0.254) (layer F.Cu) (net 16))
 (segment (start 9.25 -7.75) (end 10.72199 -9.22199) (width 0.254) (layer F.Cu) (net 16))
 (segment (start 31 -13) (end 31 -15.57202) (width 0.254) (layer F.Cu) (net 17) (status 10))
 (segment (start 28.9 -17.67202) (end 13.996086 -17.67202) (width 0.254) (layer F.Cu) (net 17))
 (segment (start 31 -15.57202) (end 28.9 -17.67202) (width 0.254) (layer F.Cu) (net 17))
 (segment (start 8.024066 -11.7) (end 2.25 -11.7) (width 0.254) (layer F.Cu) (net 17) (status 20))
 (segment (start 13.996086 -17.67202) (end 8.024066 -11.7) (width 0.254) (layer F.Cu) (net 17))
 (segment (start 31 -11) (end 31 -13) (width 0.254) (layer B.Cu) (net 17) (status 30))
 (segment (start 33 -11) (end 33 -13) (width 0.254) (layer B.Cu) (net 18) (status 30))
 (segment (start 8.182 -12.5) (end 2.25 -12.5) (width 0.254) (layer F.Cu) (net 18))
 (segment (start 13.80803 -18.12603) (end 8.182 -12.5) (width 0.254) (layer F.Cu) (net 18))
 (segment (start 30.87397 -18.12603) (end 13.80803 -18.12603) (width 0.254) (layer F.Cu) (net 18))
 (segment (start 33 -16) (end 30.87397 -18.12603) (width 0.254) (layer F.Cu) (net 18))
 (segment (start 33 -13) (end 33 -16) (width 0.254) (layer F.Cu) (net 18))
 (segment (start 8.339933 -13.3) (end 13.619973 -18.58004) (width 0.254) (layer F.Cu) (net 19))
 (segment (start 2.25 -13.3) (end 8.339933 -13.3) (width 0.254) (layer F.Cu) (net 19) (status 10))
 (segment (start 13.619973 -18.58004) (end 33.71996 -18.58004) (width 0.254) (layer F.Cu) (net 19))
 (segment (start 35 -17.3) (end 35 -13) (width 0.254) (layer F.Cu) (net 19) (status 20))
 (segment (start 33.71996 -18.58004) (end 35 -17.3) (width 0.254) (layer F.Cu) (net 19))
 (segment (start 35 -11) (end 35 -13) (width 0.254) (layer B.Cu) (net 19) (status 30))
 (segment (start 8.497867 -14.1) (end 2.25 -14.1) (width 0.254) (layer F.Cu) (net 20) (status 20))
 (segment (start 37 -17.5) (end 35.46595 -19.03405) (width 0.254) (layer F.Cu) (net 20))
 (segment (start 37 -13) (end 37 -17.5) (width 0.254) (layer F.Cu) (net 20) (status 10))
 (segment (start 37 -11) (end 37 -13) (width 0.254) (layer B.Cu) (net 20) (status 30))
 (segment (start 8.497867 -14.205801) (end 8.497867 -14.1) (width 0.254) (layer F.Cu) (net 20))
 (segment (start 13.326116 -19.03405) (end 8.497867 -14.205801) (width 0.254) (layer F.Cu) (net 20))
 (segment (start 35.46595 -19.03405) (end 13.326116 -19.03405) (width 0.254) (layer F.Cu) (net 20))
 (segment (start 2.25 -5.3) (end 6.2 -5.3) (width 0.254) (layer B.Cu) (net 3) (status 10))
 (via (at 23 -1.5) (size 0.6) (drill 0.4) (layers F.Cu B.Cu) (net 3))
 (segment (start 10 -1.5) (end 23 -1.5) (width 0.254) (layer B.Cu) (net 3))
 (segment (start 6.2 -5.3) (end 10 -1.5) (width 0.254) (layer B.Cu) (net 3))
 (segment (start 23 -1.5) (end 23 -7) (width 0.254) (layer F.Cu) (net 3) (status 20))
 (segment (start 23 -9) (end 23 -7) (width 0.254) (layer B.Cu) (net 3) (status 30))
 (segment (start 45.72 -3.81) (end 48.75 -6.84) (width 0.254) (layer B.Cu) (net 24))
 (segment (start 48.75 -6.84) (end 48.75 -16.642067) (width 0.254) (layer B.Cu) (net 24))
 (segment (start 41.402 -17.526) (end 39.43994 -19.48806) (width 0.254) (layer F.Cu) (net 23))
 (segment (start 42.672 -16.256) (end 41.402 -17.526) (width 0.254) (layer F.Cu) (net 23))
 (segment (start 44.45 -1.524) (end 42.672 -3.302) (width 0.254) (layer F.Cu) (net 23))
 (segment (start 42.672 -3.302) (end 42.672 -16.256) (width 0.254) (layer F.Cu) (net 23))
 (segment (start 47.498 -2.794) (end 46.228 -1.524) (width 0.254) (layer F.Cu) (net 23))
 (segment (start 47.498 -4.572) (end 47.498 -2.794) (width 0.254) (layer F.Cu) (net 23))
 (segment (start 46.228 -1.524) (end 44.45 -1.524) (width 0.254) (layer F.Cu) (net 23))
 (segment (start 45.72 -6.35) (end 47.498 -4.572) (width 0.254) (layer F.Cu) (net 23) (status 10))
 (segment (start 8.707934 -15.7) (end 12.950003 -19.94207) (width 0.254) (layer F.Cu) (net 24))
 (segment (start 2.25 -15.7) (end 8.707934 -15.7) (width 0.254) (layer F.Cu) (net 24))
 (segment (start 48.75 -16.642067) (end 48.75 -17.25) (width 0.254) (layer B.Cu) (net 24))
 (via (at 44.75 -19.75) (size 0.6) (drill 0.4) (layers F.Cu B.Cu) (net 24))
 (segment (start 46.25 -19.75) (end 44.75 -19.75) (width 0.254) (layer B.Cu) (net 24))
 (segment (start 48.75 -17.25) (end 46.25 -19.75) (width 0.254) (layer B.Cu) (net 24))
 (segment (start 44.875 -19.625) (end 44.75 -19.75) (width 0.254) (layer F.Cu) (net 24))
 (segment (start 46.3 -19.625) (end 44.875 -19.625) (width 0.254) (layer F.Cu) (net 24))
 (segment (start 44.55793 -19.94207) (end 44.75 -19.75) (width 0.254) (layer F.Cu) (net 24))
 (segment (start 12.950003 -19.94207) (end 44.55793 -19.94207) (width 0.254) (layer F.Cu) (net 24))
 (segment (start 46.736 -8.89) (end 45.72 -8.89) (width 0.254) (layer F.Cu) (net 22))
 (segment (start 47.752 -9.906) (end 46.736 -8.89) (width 0.254) (layer F.Cu) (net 22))
 (segment (start 47.752 -11.684) (end 47.752 -9.906) (width 0.254) (layer F.Cu) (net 22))
 (segment (start 12.761946 -20.39608) (end 49.60392 -20.39608) (width 0.254) (layer F.Cu) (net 22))
 (segment (start 8.865867 -16.5) (end 12.761946 -20.39608) (width 0.254) (layer F.Cu) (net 22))
 (segment (start 50.75 -14.682) (end 47.752 -11.684) (width 0.254) (layer F.Cu) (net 22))
 (segment (start 2.25 -16.5) (end 8.865867 -16.5) (width 0.254) (layer F.Cu) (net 22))
 (segment (start 50.375 -19.625) (end 50.5 -19.5) (width 0.254) (layer F.Cu) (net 22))
 (segment (start 49.2 -19.625) (end 50.375 -19.625) (width 0.254) (layer F.Cu) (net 22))
 (segment (start 50.5 -19.5) (end 50.75 -19.25) (width 0.254) (layer F.Cu) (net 22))
 (segment (start 49.60392 -20.39608) (end 50.5 -19.5) (width 0.254) (layer F.Cu) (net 22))
 (segment (start 50.125 -19.125) (end 50.75 -18.5) (width 0.254) (layer F.Cu) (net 22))
 (segment (start 49.2 -19.125) (end 50.125 -19.125) (width 0.254) (layer F.Cu) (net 22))
 (segment (start 50.75 -19.25) (end 50.75 -18.5) (width 0.254) (layer F.Cu) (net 22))
 (segment (start 49.875 -18.625) (end 50.75 -17.75) (width 0.254) (layer F.Cu) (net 22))
 (segment (start 50.75 -17.75) (end 50.75 -14.682) (width 0.254) (layer F.Cu) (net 22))
 (segment (start 49.2 -18.625) (end 49.875 -18.625) (width 0.254) (layer F.Cu) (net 22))
 (segment (start 50.75 -18.5) (end 50.75 -17.75) (width 0.254) (layer F.Cu) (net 22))
 (segment (start 8.4 -14.9) (end 2.25 -14.9) (width 0.254) (layer F.Cu) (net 23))
 (segment (start 8.55 -14.9) (end 8.4 -14.9) (width 0.254) (layer F.Cu) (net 23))
 (segment (start 13.13806 -19.48806) (end 8.55 -14.9) (width 0.254) (layer F.Cu) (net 23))
 (segment (start 39.43994 -19.48806) (end 13.13806 -19.48806) (width 0.254) (layer F.Cu) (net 23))
 (segment (start 39.977001 -19.122999) (end 39.61194 -19.48806) (width 0.254) (layer F.Cu) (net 23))
 (segment (start 46.222999 -19.122999) (end 39.977001 -19.122999) (width 0.254) (layer F.Cu) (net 23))
 (segment (start 46.225 -19.125) (end 46.222999 -19.122999) (width 0.254) (layer F.Cu) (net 23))
 (segment (start 46.3 -19.125) (end 46.225 -19.125) (width 0.254) (layer F.Cu) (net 23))
 (segment (start 39.61194 -19.48806) (end 39.43994 -19.48806) (width 0.254) (layer F.Cu) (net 23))
 (segment (start 41.402 -20.32) (end 12.446 -20.32) (width 0.254) (layer B.Cu) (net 21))
 (segment (start 12.446 -20.32) (end 8.626 -16.5) (width 0.254) (layer B.Cu) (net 21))
 (segment (start 8.626 -16.5) (end 2.25 -16.5) (width 0.254) (layer B.Cu) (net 21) (status 20))
 (segment (start 43.222 -18.5) (end 42.736 -18.986) (width 0.254) (layer B.Cu) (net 21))
 (segment (start 42.736 -18.986) (end 41.402 -20.32) (width 0.254) (layer B.Cu) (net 21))
 (segment (start 48.25 -13.96) (end 45.72 -11.43) (width 0.254) (layer B.Cu) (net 21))
 (segment (start 48.25 -16.5) (end 48.25 -13.96) (width 0.254) (layer B.Cu) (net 21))
 (segment (start 46.25 -18.5) (end 48.25 -16.5) (width 0.254) (layer B.Cu) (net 21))
 (segment (start 45.5 -18.5) (end 46.25 -18.5) (width 0.254) (layer B.Cu) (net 21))
 (via (at 44.7 -18.2) (size 0.6) (drill 0.4) (layers F.Cu B.Cu) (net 21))
 (segment (start 44.775 -18.125) (end 44.7 -18.2) (width 0.254) (layer F.Cu) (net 21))
 (segment (start 46.3 -18.125) (end 44.775 -18.125) (width 0.254) (layer F.Cu) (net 21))
 (segment (start 44.7 -18.2) (end 44.4 -18.5) (width 0.254) (layer B.Cu) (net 21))
 (segment (start 44.4 -18.5) (end 44.2 -18.5) (width 0.254) (layer B.Cu) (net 21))
 (segment (start 44.2 -18.5) (end 43.222 -18.5) (width 0.254) (layer B.Cu) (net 21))
 (segment (start 45.5 -18.5) (end 44.2 -18.5) (width 0.254) (layer B.Cu) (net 21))
 (segment (start 48.5 -17.5) (end 48.5 -16.75) (width 0.254) (layer F.Cu) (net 26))
 (segment (start 49.125 -18.125) (end 48.5 -17.5) (width 0.254) (layer F.Cu) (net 26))
 (segment (start 49.2 -18.125) (end 49.125 -18.125) (width 0.254) (layer F.Cu) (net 26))
 (via (at 44.8 -16.7) (size 0.6) (drill 0.4) (layers F.Cu B.Cu) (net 25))
 (segment (start 44.85 -16.75) (end 44.8 -16.7) (width 0.254) (layer F.Cu) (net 25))
 (segment (start 47 -16.75) (end 44.85 -16.75) (width 0.254) (layer F.Cu) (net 25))
 (segment (start 8.468066 -15.7) (end 2.25 -15.7) (width 0.254) (layer B.Cu) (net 25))
 (segment (start 12.634056 -19.86599) (end 8.468066 -15.7) (width 0.254) (layer B.Cu) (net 25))
 (segment (start 40.63401 -19.86599) (end 12.634056 -19.86599) (width 0.254) (layer B.Cu) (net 25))
 (segment (start 43.8 -16.7) (end 40.63401 -19.86599) (width 0.254) (layer B.Cu) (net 25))
 (segment (start 44.8 -16.7) (end 43.8 -16.7) (width 0.254) (layer B.Cu) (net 25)))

